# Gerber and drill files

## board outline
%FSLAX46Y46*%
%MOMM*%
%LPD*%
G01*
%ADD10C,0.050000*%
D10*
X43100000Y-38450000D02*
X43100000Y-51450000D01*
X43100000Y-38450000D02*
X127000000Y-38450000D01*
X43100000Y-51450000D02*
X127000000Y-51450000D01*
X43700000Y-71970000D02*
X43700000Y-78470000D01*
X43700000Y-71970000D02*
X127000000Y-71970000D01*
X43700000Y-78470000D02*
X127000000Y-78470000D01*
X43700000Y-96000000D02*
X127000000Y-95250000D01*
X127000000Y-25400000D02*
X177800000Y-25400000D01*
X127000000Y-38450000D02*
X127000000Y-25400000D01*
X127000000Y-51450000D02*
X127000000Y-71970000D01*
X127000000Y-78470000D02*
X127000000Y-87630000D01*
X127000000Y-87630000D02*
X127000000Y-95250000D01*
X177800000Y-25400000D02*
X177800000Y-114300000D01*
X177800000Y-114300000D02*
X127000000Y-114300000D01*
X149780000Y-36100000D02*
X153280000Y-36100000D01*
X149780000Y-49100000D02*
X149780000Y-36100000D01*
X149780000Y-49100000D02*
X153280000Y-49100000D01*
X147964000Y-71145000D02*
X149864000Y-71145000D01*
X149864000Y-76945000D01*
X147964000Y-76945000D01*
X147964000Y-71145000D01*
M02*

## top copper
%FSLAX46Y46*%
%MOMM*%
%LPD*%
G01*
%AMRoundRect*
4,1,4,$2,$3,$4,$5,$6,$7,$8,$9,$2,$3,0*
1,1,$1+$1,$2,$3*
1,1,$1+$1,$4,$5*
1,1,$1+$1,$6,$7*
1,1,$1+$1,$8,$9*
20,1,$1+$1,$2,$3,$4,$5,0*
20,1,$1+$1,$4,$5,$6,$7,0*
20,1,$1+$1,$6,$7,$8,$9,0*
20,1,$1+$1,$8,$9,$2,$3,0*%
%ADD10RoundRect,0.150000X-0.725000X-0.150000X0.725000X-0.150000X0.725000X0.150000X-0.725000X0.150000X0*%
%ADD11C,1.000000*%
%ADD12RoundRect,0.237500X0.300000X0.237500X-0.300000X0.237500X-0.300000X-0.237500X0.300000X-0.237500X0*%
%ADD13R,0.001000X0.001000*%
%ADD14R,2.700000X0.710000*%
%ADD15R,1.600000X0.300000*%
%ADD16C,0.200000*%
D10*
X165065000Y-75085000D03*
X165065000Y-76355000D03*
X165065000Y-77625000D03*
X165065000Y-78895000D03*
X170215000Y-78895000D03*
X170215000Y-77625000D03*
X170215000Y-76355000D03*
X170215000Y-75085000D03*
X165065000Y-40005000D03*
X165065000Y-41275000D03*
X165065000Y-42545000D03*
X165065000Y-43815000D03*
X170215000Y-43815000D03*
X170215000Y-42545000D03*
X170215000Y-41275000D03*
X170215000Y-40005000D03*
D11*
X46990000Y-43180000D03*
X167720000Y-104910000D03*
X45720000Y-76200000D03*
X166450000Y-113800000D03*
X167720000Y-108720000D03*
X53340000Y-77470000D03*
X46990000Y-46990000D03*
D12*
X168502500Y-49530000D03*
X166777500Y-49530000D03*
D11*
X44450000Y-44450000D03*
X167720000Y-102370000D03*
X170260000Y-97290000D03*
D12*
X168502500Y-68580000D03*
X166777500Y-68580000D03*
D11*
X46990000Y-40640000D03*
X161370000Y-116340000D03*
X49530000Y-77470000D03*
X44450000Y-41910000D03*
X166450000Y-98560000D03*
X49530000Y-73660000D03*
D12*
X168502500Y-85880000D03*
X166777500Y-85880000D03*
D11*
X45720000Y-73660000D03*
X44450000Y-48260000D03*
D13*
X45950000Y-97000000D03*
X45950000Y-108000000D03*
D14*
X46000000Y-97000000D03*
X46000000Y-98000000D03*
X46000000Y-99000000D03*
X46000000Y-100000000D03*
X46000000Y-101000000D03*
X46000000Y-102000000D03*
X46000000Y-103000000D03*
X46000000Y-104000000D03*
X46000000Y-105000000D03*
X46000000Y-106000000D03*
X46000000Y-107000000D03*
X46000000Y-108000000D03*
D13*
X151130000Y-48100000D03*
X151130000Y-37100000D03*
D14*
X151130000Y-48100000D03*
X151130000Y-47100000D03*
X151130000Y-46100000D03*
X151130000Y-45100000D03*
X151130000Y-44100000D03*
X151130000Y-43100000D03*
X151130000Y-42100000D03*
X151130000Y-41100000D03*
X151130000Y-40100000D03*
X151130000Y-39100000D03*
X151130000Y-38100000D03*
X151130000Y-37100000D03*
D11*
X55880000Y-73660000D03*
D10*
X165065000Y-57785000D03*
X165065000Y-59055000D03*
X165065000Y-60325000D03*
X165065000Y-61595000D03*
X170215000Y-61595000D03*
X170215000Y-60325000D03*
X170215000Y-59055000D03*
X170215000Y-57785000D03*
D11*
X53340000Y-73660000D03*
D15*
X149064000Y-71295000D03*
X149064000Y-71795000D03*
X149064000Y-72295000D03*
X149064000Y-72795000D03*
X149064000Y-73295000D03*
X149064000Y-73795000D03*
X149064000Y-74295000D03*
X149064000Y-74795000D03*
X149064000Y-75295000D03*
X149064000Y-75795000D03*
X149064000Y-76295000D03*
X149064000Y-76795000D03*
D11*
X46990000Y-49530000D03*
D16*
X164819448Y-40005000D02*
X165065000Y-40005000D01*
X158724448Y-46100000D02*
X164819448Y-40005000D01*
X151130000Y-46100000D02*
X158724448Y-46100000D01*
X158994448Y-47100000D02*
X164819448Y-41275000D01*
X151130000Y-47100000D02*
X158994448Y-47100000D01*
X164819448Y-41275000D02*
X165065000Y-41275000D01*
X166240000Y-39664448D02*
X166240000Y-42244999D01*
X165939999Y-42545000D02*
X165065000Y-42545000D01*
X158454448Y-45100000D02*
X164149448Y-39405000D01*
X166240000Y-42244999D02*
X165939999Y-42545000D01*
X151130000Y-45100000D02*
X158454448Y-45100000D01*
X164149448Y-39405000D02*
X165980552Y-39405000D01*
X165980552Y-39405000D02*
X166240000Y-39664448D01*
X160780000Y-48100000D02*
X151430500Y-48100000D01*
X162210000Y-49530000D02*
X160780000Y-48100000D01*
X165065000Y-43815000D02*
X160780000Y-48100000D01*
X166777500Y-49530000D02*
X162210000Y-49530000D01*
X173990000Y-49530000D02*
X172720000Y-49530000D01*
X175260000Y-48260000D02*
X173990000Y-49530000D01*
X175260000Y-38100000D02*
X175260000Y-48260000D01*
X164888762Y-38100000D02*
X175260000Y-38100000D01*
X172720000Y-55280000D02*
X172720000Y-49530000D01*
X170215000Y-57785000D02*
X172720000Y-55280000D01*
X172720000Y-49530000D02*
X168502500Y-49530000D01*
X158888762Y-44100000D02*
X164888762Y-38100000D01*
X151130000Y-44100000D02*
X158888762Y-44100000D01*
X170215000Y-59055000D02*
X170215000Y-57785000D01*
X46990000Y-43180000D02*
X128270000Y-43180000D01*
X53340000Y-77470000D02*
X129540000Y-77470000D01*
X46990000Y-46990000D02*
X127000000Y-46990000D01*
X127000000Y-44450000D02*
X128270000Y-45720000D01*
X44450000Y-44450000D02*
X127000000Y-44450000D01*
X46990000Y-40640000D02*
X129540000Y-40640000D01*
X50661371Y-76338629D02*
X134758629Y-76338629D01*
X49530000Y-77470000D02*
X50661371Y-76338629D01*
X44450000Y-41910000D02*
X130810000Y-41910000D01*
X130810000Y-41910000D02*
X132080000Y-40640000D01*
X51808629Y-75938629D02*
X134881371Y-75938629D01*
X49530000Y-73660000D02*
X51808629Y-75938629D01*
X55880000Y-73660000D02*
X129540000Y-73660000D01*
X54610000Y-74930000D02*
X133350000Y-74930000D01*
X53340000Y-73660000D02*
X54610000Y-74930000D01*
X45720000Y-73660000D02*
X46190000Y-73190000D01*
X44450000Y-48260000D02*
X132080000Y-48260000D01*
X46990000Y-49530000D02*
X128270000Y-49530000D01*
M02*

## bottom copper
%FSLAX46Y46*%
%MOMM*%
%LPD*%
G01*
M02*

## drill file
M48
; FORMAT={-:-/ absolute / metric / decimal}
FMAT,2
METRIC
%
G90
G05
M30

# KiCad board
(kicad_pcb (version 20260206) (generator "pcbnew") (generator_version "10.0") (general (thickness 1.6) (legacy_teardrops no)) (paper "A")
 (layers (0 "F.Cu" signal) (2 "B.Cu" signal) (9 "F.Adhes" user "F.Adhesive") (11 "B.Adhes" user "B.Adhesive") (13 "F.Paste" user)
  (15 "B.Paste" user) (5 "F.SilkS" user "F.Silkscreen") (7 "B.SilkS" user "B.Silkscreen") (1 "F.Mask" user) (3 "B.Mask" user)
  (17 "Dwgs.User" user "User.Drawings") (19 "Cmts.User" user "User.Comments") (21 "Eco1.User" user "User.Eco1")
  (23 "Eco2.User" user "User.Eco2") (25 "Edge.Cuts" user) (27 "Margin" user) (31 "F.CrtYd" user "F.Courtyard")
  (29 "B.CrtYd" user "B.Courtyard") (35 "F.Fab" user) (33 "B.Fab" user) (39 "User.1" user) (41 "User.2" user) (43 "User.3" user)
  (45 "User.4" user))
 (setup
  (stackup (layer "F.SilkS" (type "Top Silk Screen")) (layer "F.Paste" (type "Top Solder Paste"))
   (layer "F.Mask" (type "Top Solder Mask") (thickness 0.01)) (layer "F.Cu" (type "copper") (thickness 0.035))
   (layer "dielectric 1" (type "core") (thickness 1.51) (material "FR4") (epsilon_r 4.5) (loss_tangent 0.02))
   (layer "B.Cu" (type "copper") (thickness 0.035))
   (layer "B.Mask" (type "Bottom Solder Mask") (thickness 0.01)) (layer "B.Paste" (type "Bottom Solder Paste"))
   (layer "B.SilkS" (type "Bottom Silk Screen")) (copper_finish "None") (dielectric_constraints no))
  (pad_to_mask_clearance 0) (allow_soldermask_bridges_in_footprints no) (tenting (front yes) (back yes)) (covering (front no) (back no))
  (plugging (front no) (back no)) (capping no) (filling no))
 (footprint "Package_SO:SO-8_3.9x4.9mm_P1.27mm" (layer "F.Cu") (at 167.64 76.99)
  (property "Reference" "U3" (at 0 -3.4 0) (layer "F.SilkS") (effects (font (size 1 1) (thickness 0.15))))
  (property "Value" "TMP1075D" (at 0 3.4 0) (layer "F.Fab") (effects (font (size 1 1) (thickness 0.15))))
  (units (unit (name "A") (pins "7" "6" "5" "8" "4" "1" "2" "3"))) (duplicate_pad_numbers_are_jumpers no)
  (pad "1" smd roundrect (at -2.575 -1.905) (size 1.75 0.6) (layers "F.Cu" "F.Mask" "F.Paste") (roundrect_rratio 0.25) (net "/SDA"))
  (pad "2" smd roundrect (at -2.575 -0.635) (size 1.75 0.6) (layers "F.Cu" "F.Mask" "F.Paste") (roundrect_rratio 0.25) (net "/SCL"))
  (pad "3" smd roundrect (at -2.575 0.635) (size 1.75 0.6) (layers "F.Cu" "F.Mask" "F.Paste") (roundrect_rratio 0.25) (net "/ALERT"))
  (pad "4" smd roundrect (at -2.575 1.905) (size 1.75 0.6) (layers "F.Cu" "F.Mask" "F.Paste") (roundrect_rratio 0.25) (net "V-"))
  (pad "5" smd roundrect (at 2.575 1.905) (size 1.75 0.6) (layers "F.Cu" "F.Mask" "F.Paste") (roundrect_rratio 0.25) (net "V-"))
  (pad "6" smd roundrect (at 2.575 0.635) (size 1.75 0.6) (layers "F.Cu" "F.Mask" "F.Paste") (roundrect_rratio 0.25) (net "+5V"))
  (pad "7" smd roundrect (at 2.575 -0.635) (size 1.75 0.6) (layers "F.Cu" "F.Mask" "F.Paste") (roundrect_rratio 0.25) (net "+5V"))
  (pad "8" smd roundrect (at 2.575 -1.905) (size 1.75 0.6) (layers "F.Cu" "F.Mask" "F.Paste") (roundrect_rratio 0.25) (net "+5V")))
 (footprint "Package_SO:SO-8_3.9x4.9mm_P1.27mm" (layer "F.Cu") (at 167.64 41.91)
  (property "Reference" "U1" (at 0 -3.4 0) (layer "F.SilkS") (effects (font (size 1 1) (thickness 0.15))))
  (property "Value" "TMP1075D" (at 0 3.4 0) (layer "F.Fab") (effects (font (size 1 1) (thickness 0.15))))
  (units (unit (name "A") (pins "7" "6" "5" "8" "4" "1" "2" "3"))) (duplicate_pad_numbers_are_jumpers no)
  (pad "1" smd roundrect (at -2.575 -1.905) (size 1.75 0.6) (layers "F.Cu" "F.Mask" "F.Paste") (roundrect_rratio 0.25) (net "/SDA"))
  (pad "2" smd roundrect (at -2.575 -0.635) (size 1.75 0.6) (layers "F.Cu" "F.Mask" "F.Paste") (roundrect_rratio 0.25) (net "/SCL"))
  (pad "3" smd roundrect (at -2.575 0.635) (size 1.75 0.6) (layers "F.Cu" "F.Mask" "F.Paste") (roundrect_rratio 0.25) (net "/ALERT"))
  (pad "4" smd roundrect (at -2.575 1.905) (size 1.75 0.6) (layers "F.Cu" "F.Mask" "F.Paste") (roundrect_rratio 0.25) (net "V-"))
  (pad "5" smd roundrect (at 2.575 1.905) (size 1.75 0.6) (layers "F.Cu" "F.Mask" "F.Paste") (roundrect_rratio 0.25) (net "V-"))
  (pad "6" smd roundrect (at 2.575 0.635) (size 1.75 0.6) (layers "F.Cu" "F.Mask" "F.Paste") (roundrect_rratio 0.25) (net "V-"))
  (pad "7" smd roundrect (at 2.575 -0.635) (size 1.75 0.6) (layers "F.Cu" "F.Mask" "F.Paste") (roundrect_rratio 0.25) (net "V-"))
  (pad "8" smd roundrect (at 2.575 -1.905) (size 1.75 0.6) (layers "F.Cu" "F.Mask" "F.Paste") (roundrect_rratio 0.25) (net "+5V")))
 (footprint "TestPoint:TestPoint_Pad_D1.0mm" (layer "F.Cu") (at 46.99 43.18)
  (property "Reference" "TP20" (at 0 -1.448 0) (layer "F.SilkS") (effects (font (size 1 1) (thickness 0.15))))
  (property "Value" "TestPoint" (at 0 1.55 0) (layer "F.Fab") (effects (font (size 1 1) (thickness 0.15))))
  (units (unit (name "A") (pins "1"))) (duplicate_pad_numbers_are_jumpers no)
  (pad "1" smd circle (at 0 0) (size 1 1) (layers "F.Cu" "F.Mask") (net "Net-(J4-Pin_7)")))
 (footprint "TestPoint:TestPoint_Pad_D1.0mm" (layer "F.Cu") (at 167.72 104.91 90)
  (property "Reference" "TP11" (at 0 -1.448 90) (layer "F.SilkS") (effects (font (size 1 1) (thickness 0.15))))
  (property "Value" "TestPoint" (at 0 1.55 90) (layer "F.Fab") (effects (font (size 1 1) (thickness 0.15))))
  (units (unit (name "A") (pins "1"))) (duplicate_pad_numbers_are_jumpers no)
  (pad "1" smd circle (at 0 0 90) (size 1 1) (layers "F.Cu" "F.Mask") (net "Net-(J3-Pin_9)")))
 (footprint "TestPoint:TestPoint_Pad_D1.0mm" (layer "F.Cu") (at 45.72 76.2)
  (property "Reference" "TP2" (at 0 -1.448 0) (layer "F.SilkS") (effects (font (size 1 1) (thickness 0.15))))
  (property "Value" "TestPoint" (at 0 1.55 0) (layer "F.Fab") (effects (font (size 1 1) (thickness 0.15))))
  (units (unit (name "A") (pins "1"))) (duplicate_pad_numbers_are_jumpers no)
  (pad "1" smd circle (at 0 0) (size 1 1) (layers "F.Cu" "F.Mask") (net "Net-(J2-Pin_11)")))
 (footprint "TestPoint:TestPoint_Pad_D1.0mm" (layer "F.Cu") (at 166.45 113.8 90)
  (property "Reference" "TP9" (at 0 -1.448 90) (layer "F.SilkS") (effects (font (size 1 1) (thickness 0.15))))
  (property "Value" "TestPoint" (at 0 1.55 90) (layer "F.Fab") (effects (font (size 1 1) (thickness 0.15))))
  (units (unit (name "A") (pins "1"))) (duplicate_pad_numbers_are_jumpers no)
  (pad "1" smd circle (at 0 0 90) (size 1 1) (layers "F.Cu" "F.Mask") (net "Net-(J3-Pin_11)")))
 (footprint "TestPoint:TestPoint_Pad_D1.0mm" (layer "F.Cu") (at 167.72 108.72 90)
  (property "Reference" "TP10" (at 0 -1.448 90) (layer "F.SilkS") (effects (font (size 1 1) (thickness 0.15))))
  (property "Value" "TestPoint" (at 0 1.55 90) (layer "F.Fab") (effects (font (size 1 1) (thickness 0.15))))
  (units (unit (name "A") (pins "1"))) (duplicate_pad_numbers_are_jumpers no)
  (pad "1" smd circle (at 0 0 90) (size 1 1) (layers "F.Cu" "F.Mask") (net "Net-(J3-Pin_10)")))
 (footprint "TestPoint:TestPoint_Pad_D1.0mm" (layer "F.Cu") (at 53.34 77.47)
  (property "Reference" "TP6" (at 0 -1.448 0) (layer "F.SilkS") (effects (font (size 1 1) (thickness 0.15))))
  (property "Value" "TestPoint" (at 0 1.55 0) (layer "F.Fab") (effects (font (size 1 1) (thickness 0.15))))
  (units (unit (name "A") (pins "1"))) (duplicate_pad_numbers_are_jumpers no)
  (pad "1" smd circle (at 0 0) (size 1 1) (layers "F.Cu" "F.Mask") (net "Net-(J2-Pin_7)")))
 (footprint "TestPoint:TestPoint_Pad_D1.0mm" (layer "F.Cu") (at 46.99 46.99)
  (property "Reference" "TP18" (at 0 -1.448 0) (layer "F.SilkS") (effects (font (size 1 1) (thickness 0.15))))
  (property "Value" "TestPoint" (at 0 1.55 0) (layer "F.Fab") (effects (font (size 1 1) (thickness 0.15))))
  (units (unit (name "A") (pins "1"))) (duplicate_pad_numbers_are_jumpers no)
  (pad "1" smd circle (at 0 0) (size 1 1) (layers "F.Cu" "F.Mask") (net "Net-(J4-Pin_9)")))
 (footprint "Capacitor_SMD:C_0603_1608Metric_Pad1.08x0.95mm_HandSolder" (layer "F.Cu") (at 167.64 49.53 180)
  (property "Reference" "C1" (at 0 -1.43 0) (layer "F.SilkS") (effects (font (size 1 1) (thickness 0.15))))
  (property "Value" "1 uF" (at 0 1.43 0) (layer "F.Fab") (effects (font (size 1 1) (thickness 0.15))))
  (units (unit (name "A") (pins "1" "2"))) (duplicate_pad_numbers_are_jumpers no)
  (pad "1" smd roundrect (at -0.8625 0 180) (size 1.075 0.95) (layers "F.Cu" "F.Mask" "F.Paste") (roundrect_rratio 0.25) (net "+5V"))
  (pad "2" smd roundrect (at 0.8625 0 180) (size 1.075 0.95) (layers "F.Cu" "F.Mask" "F.Paste") (roundrect_rratio 0.25) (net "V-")))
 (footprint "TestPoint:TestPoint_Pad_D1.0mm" (layer "F.Cu") (at 44.45 44.45)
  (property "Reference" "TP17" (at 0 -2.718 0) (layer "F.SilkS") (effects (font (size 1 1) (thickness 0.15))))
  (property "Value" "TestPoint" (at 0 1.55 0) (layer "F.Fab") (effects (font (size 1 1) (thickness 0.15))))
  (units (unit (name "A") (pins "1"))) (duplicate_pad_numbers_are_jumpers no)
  (pad "1" smd circle (at 0 0) (size 1 1) (layers "F.Cu" "F.Mask") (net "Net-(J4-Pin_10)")))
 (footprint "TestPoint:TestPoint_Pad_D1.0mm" (layer "F.Cu") (at 167.72 102.37 90)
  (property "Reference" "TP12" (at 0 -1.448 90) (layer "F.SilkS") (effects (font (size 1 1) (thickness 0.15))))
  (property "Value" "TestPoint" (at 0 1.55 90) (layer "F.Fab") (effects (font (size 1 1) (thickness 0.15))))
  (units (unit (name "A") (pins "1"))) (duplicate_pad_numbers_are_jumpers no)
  (pad "1" smd circle (at 0 0 90) (size 1 1) (layers "F.Cu" "F.Mask") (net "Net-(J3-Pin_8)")))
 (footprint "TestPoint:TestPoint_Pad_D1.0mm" (layer "F.Cu") (at 170.26 97.29 90)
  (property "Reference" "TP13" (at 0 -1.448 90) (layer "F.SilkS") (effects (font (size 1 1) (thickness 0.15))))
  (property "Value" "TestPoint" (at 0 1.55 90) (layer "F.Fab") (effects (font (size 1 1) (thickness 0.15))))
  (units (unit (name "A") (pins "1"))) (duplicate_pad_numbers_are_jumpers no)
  (pad "1" smd circle (at 0 0 90) (size 1 1) (layers "F.Cu" "F.Mask") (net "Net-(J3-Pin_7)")))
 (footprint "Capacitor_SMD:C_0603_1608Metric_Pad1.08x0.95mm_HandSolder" (layer "F.Cu") (at 167.64 68.58 180)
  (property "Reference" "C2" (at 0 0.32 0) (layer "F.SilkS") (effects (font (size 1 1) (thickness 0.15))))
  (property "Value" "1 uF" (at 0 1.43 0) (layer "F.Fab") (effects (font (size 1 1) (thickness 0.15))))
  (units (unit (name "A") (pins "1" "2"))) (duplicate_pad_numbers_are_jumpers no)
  (pad "1" smd roundrect (at -0.8625 0 180) (size 1.075 0.95) (layers "F.Cu" "F.Mask" "F.Paste") (roundrect_rratio 0.25) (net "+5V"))
  (pad "2" smd roundrect (at 0.8625 0 180) (size 1.075 0.95) (layers "F.Cu" "F.Mask" "F.Paste") (roundrect_rratio 0.25) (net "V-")))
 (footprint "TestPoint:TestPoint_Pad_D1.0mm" (layer "F.Cu") (at 46.99 40.64)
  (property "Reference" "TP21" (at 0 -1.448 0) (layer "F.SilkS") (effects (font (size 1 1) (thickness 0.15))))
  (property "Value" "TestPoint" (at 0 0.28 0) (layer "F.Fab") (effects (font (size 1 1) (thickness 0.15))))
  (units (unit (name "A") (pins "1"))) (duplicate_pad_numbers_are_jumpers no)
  (pad "1" smd circle (at 0 0) (size 1 1) (layers "F.Cu" "F.Mask") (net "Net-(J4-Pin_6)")))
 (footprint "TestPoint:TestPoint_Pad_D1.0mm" (layer "F.Cu") (at 161.37 116.34 90)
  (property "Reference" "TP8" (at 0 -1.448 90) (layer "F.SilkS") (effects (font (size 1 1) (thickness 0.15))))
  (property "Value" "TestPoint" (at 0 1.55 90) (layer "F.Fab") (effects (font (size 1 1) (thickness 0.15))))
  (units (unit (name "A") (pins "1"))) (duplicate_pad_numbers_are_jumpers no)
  (pad "1" smd circle (at 0 0 90) (size 1 1) (layers "F.Cu" "F.Mask") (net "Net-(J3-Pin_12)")))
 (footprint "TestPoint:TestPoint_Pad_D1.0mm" (layer "F.Cu") (at 49.53 77.47)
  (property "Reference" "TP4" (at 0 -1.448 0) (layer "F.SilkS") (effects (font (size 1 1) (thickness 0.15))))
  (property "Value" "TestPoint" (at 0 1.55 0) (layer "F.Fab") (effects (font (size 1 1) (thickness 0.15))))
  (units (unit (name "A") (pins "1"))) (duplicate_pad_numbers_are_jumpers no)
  (pad "1" smd circle (at 0 0) (size 1 1) (layers "F.Cu" "F.Mask") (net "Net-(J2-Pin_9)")))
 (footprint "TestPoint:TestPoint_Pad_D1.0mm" (layer "F.Cu") (at 44.45 41.91)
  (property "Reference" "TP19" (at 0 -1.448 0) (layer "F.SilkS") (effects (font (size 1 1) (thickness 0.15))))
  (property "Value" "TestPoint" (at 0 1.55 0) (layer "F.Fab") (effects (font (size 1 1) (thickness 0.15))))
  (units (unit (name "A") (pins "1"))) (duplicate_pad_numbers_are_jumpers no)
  (pad "1" smd circle (at 0 0) (size 1 1) (layers "F.Cu" "F.Mask") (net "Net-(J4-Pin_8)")))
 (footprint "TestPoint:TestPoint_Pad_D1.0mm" (layer "F.Cu") (at 166.45 98.56 90)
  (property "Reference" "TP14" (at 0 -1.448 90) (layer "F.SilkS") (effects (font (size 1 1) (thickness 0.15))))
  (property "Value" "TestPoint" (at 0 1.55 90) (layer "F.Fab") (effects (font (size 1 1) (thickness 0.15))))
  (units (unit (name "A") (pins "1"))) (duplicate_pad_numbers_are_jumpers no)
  (pad "1" smd circle (at 0 0 90) (size 1 1) (layers "F.Cu" "F.Mask") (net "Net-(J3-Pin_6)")))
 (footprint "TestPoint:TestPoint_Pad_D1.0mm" (layer "F.Cu") (at 49.53 73.66)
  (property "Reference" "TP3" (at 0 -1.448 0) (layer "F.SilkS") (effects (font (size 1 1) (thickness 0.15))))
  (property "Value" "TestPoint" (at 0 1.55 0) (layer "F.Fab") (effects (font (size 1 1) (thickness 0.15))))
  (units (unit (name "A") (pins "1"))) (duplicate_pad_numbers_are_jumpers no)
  (pad "1" smd circle (at 0 0) (size 1 1) (layers "F.Cu" "F.Mask") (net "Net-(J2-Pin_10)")))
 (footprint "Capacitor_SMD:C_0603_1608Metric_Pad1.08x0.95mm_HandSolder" (layer "F.Cu") (at 167.64 85.88 180)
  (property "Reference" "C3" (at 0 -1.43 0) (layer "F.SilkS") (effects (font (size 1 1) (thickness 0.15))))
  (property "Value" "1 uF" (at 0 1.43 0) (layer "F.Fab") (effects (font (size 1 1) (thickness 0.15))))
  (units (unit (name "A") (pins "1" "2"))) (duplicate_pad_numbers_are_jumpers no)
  (pad "1" smd roundrect (at -0.8625 0 180) (size 1.075 0.95) (layers "F.Cu" "F.Mask" "F.Paste") (roundrect_rratio 0.25) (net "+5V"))
  (pad "2" smd roundrect (at 0.8625 0 180) (size 1.075 0.95) (layers "F.Cu" "F.Mask" "F.Paste") (roundrect_rratio 0.25) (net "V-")))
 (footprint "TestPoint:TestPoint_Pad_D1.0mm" (layer "F.Cu") (at 45.72 73.66)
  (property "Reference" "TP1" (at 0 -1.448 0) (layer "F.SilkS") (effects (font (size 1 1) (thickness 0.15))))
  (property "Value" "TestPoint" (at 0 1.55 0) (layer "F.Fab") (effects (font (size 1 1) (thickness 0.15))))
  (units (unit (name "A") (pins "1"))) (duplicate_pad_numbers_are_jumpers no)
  (pad "1" smd circle (at 0 0) (size 1 1) (layers "F.Cu" "F.Mask") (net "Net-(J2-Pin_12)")))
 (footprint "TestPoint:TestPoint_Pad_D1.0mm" (layer "F.Cu") (at 44.45 48.26)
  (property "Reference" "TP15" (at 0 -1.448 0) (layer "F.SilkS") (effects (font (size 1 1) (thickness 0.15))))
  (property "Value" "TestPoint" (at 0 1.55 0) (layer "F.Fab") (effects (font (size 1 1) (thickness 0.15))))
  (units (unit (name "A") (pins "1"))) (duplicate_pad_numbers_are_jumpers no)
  (pad "1" smd circle (at 0 0) (size 1 1) (layers "F.Cu" "F.Mask") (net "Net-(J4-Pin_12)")))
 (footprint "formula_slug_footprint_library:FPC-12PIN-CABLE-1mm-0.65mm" (layer "F.Cu") (at 47.35 102.5 -90)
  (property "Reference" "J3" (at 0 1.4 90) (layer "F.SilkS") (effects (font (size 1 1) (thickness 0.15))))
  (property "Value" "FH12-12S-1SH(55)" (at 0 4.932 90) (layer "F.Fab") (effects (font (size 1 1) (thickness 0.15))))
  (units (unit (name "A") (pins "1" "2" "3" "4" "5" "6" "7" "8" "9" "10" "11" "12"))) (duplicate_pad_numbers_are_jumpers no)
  (pad "0" smd rect (at -5.5 1.4 270) (size 0.001 0.001) (layers "F.Cu" "F.Mask" "F.Paste") (thermal_bridge_angle 45))
  (pad "0" smd rect (at 5.5 1.4 270) (size 0.001 0.001) (layers "F.Cu" "F.Mask" "F.Paste") (thermal_bridge_angle 45))
  (pad "1" smd rect (at -5.5 1.35 270) (size 0.71 2.7) (layers "F.Cu" "F.Mask" "F.Paste") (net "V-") (thermal_bridge_angle 45))
  (pad "2" smd rect (at -4.5 1.35 270) (size 0.71 2.7) (layers "F.Cu" "F.Mask" "F.Paste") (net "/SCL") (thermal_bridge_angle 45))
  (pad "3" smd rect (at -3.5 1.35 270) (size 0.71 2.7) (layers "F.Cu" "F.Mask" "F.Paste") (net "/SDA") (thermal_bridge_angle 45))
  (pad "4" smd rect (at -2.5 1.35 270) (size 0.71 2.7) (layers "F.Cu" "F.Mask" "F.Paste") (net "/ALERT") (thermal_bridge_angle 45))
  (pad "5" smd rect (at -1.5 1.35 270) (size 0.71 2.7) (layers "F.Cu" "F.Mask" "F.Paste") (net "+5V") (thermal_bridge_angle 45))
  (pad "6" smd rect (at -0.5 1.35 270) (size 0.71 2.7) (layers "F.Cu" "F.Mask" "F.Paste") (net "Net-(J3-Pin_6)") (thermal_bridge_angle 45))
  (pad "7" smd rect (at 0.5 1.35 270) (size 0.71 2.7) (layers "F.Cu" "F.Mask" "F.Paste") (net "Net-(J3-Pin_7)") (thermal_bridge_angle 45))
  (pad "8" smd rect (at 1.5 1.35 270) (size 0.71 2.7) (layers "F.Cu" "F.Mask" "F.Paste") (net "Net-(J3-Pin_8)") (thermal_bridge_angle 45))
  (pad "9" smd rect (at 2.5 1.35 270) (size 0.71 2.7) (layers "F.Cu" "F.Mask" "F.Paste") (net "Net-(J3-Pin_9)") (thermal_bridge_angle 45))
  (pad "10" smd rect (at 3.5 1.35 270) (size 0.71 2.7) (layers "F.Cu" "F.Mask" "F.Paste") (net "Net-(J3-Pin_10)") (thermal_bridge_angle 45))
  (pad "11" smd rect (at 4.5 1.35 270) (size 0.71 2.7) (layers "F.Cu" "F.Mask" "F.Paste") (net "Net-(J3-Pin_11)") (thermal_bridge_angle 45))
  (pad "12" smd rect (at 5.5 1.35 270) (size 0.71 2.7) (layers "F.Cu" "F.Mask" "F.Paste") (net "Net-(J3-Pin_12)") (thermal_bridge_angle 45)))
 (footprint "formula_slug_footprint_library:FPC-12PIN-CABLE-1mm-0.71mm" (layer "F.Cu") (at 149.78 42.6 90)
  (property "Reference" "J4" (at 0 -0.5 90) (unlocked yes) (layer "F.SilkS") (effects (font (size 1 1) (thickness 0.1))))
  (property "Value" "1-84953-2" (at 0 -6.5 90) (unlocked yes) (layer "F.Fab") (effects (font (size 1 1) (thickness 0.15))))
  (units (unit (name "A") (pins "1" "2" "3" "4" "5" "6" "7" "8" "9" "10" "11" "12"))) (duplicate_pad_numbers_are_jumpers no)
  (fp_line (start 6.5 0) (end 6.5 3.5) (stroke (width 0.05) (type solid)) (layer "Edge.Cuts"))
  (fp_line (start -6.5 0) (end 6.5 0) (stroke (width 0.05) (type solid)) (layer "Edge.Cuts"))
  (fp_line (start -6.5 0) (end -6.5 3.5) (stroke (width 0.05) (type solid)) (layer "Edge.Cuts"))
  (pad "0" smd rect (at -5.5 1.35 90) (size 0.001 0.001) (layers "F.Cu" "F.Mask" "F.Paste") (thermal_bridge_angle 45))
  (pad "0" smd rect (at 5.5 1.35 90) (size 0.001 0.001) (layers "F.Cu" "F.Mask" "F.Paste") (thermal_bridge_angle 45))
  (pad "1" smd rect (at -5.5 1.35 90) (size 0.71 2.7) (layers "F.Cu" "F.Mask" "F.Paste") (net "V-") (thermal_bridge_angle 45))
  (pad "2" smd rect (at -4.5 1.35 90) (size 0.71 2.7) (layers "F.Cu" "F.Mask" "F.Paste") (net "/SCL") (thermal_bridge_angle 45))
  (pad "3" smd rect (at -3.5 1.35 90) (size 0.71 2.7) (layers "F.Cu" "F.Mask" "F.Paste") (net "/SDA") (thermal_bridge_angle 45))
  (pad "4" smd rect (at -2.5 1.35 90) (size 0.71 2.7) (layers "F.Cu" "F.Mask" "F.Paste") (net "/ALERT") (thermal_bridge_angle 45))
  (pad "5" smd rect (at -1.5 1.35 90) (size 0.71 2.7) (layers "F.Cu" "F.Mask" "F.Paste") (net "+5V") (thermal_bridge_angle 45))
  (pad "6" smd rect (at -0.5 1.35 90) (size 0.71 2.7) (layers "F.Cu" "F.Mask" "F.Paste") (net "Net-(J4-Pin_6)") (thermal_bridge_angle 45))
  (pad "7" smd rect (at 0.5 1.35 90) (size 0.71 2.7) (layers "F.Cu" "F.Mask" "F.Paste") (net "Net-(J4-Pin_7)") (thermal_bridge_angle 45))
  (pad "8" smd rect (at 1.5 1.35 90) (size 0.71 2.7) (layers "F.Cu" "F.Mask" "F.Paste") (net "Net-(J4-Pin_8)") (thermal_bridge_angle 45))
  (pad "9" smd rect (at 2.5 1.35 90) (size 0.71 2.7) (layers "F.Cu" "F.Mask" "F.Paste") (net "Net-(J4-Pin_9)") (thermal_bridge_angle 45))
  (pad "10" smd rect (at 3.5 1.35 90) (size 0.71 2.7) (layers "F.Cu" "F.Mask" "F.Paste") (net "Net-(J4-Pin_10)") (thermal_bridge_angle 45))
  (pad "11" smd rect (at 4.5 1.35 90) (size 0.71 2.7) (layers "F.Cu" "F.Mask" "F.Paste") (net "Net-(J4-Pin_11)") (thermal_bridge_angle 45))
  (pad "12" smd rect (at 5.5 1.35 90) (size 0.71 2.7) (layers "F.Cu" "F.Mask" "F.Paste") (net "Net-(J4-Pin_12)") (thermal_bridge_angle 45)))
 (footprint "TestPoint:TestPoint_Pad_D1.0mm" (layer "F.Cu") (at 55.88 73.66)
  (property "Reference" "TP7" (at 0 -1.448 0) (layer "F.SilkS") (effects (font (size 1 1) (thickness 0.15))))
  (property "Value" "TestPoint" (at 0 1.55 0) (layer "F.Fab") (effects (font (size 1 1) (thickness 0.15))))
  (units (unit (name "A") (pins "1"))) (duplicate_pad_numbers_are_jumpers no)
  (pad "1" smd circle (at 0 0) (size 1 1) (layers "F.Cu" "F.Mask") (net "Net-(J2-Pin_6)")))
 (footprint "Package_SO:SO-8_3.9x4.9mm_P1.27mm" (layer "F.Cu") (at 167.64 59.69)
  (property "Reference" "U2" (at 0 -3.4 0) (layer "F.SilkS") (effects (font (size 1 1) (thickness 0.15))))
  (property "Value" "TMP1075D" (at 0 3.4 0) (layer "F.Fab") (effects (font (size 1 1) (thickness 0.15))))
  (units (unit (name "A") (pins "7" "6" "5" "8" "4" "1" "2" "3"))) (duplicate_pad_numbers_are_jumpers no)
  (pad "1" smd roundrect (at -2.575 -1.905) (size 1.75 0.6) (layers "F.Cu" "F.Mask" "F.Paste") (roundrect_rratio 0.25) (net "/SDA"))
  (pad "2" smd roundrect (at -2.575 -0.635) (size 1.75 0.6) (layers "F.Cu" "F.Mask" "F.Paste") (roundrect_rratio 0.25) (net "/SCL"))
  (pad "3" smd roundrect (at -2.575 0.635) (size 1.75 0.6) (layers "F.Cu" "F.Mask" "F.Paste") (roundrect_rratio 0.25) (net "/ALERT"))
  (pad "4" smd roundrect (at -2.575 1.905) (size 1.75 0.6) (layers "F.Cu" "F.Mask" "F.Paste") (roundrect_rratio 0.25) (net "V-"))
  (pad "5" smd roundrect (at 2.575 1.905) (size 1.75 0.6) (layers "F.Cu" "F.Mask" "F.Paste") (roundrect_rratio 0.25) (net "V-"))
  (pad "6" smd roundrect (at 2.575 0.635) (size 1.75 0.6) (layers "F.Cu" "F.Mask" "F.Paste") (roundrect_rratio 0.25) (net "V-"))
  (pad "7" smd roundrect (at 2.575 -0.635) (size 1.75 0.6) (layers "F.Cu" "F.Mask" "F.Paste") (roundrect_rratio 0.25) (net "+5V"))
  (pad "8" smd roundrect (at 2.575 -1.905) (size 1.75 0.6) (layers "F.Cu" "F.Mask" "F.Paste") (roundrect_rratio 0.25) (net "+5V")))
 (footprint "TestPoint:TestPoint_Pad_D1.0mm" (layer "F.Cu") (at 53.34 73.66)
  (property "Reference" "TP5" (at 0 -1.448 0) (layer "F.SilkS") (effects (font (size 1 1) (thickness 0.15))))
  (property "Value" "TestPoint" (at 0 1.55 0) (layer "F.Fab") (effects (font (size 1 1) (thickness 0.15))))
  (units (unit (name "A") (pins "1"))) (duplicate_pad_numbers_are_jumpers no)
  (pad "1" smd circle (at 0 0) (size 1 1) (layers "F.Cu" "F.Mask") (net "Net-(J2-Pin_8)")))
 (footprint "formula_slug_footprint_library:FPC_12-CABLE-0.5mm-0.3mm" (layer "F.Cu") (at 149.864 74.045 -90)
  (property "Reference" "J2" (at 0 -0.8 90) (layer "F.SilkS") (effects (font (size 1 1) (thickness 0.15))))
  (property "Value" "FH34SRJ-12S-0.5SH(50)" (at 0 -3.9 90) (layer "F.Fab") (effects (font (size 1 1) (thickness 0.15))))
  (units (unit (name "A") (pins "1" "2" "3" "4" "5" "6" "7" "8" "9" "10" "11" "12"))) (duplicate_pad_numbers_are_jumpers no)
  (fp_rect (start -2.9 0) (end 2.9 1.9) (stroke (width 0.05) (type solid)) (fill no) (layer "Edge.Cuts"))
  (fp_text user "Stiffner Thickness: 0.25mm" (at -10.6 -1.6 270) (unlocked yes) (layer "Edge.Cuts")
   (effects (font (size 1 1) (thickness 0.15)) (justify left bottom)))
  (pad "1" smd rect (at -2.75 0.8 270) (size 0.3 1.6) (layers "F.Cu" "F.Mask" "F.Paste") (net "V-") (thermal_bridge_angle 45))
  (pad "2" smd rect (at -2.25 0.8 270) (size 0.3 1.6) (layers "F.Cu" "F.Mask" "F.Paste") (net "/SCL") (thermal_bridge_angle 45))
  (pad "3" smd rect (at -1.75 0.8 270) (size 0.3 1.6) (layers "F.Cu" "F.Mask" "F.Paste") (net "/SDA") (thermal_bridge_angle 45))
  (pad "4" smd rect (at -1.25 0.8 270) (size 0.3 1.6) (layers "F.Cu" "F.Mask" "F.Paste") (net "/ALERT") (thermal_bridge_angle 45))
  (pad "5" smd rect (at -0.75 0.8 270) (size 0.3 1.6) (layers "F.Cu" "F.Mask" "F.Paste") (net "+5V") (thermal_bridge_angle 45))
  (pad "6" smd rect (at -0.25 0.8 270) (size 0.3 1.6) (layers "F.Cu" "F.Mask" "F.Paste") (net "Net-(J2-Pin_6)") (thermal_bridge_angle 45))
  (pad "7" smd rect (at 0.25 0.8 270) (size 0.3 1.6) (layers "F.Cu" "F.Mask" "F.Paste") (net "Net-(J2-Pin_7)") (thermal_bridge_angle 45))
  (pad "8" smd rect (at 0.75 0.8 270) (size 0.3 1.6) (layers "F.Cu" "F.Mask" "F.Paste") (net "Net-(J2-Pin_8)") (thermal_bridge_angle 45))
  (pad "9" smd rect (at 1.25 0.8 270) (size 0.3 1.6) (layers "F.Cu" "F.Mask" "F.Paste") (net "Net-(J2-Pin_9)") (thermal_bridge_angle 45))
  (pad "10" smd rect (at 1.75 0.8 270) (size 0.3 1.6) (layers "F.Cu" "F.Mask" "F.Paste") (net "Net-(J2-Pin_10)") (thermal_bridge_angle 45))
  (pad "11" smd rect (at 2.25 0.8 270) (size 0.3 1.6) (layers "F.Cu" "F.Mask" "F.Paste") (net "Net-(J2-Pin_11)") (thermal_bridge_angle 45))
  (pad "12" smd rect (at 2.75 0.8 270) (size 0.3 1.6) (layers "F.Cu" "F.Mask" "F.Paste") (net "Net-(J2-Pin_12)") (thermal_bridge_angle 45)))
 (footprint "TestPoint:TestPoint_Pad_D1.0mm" (layer "F.Cu") (at 46.99 49.53)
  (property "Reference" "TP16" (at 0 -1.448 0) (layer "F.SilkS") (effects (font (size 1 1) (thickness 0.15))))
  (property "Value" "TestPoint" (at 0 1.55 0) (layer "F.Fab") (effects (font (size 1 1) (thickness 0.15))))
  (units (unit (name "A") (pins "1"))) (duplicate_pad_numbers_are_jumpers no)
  (pad "1" smd circle (at 0 0) (size 1 1) (layers "F.Cu" "F.Mask") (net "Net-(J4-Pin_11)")))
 (gr_line (start 43.1 38.45) (end 43.1 51.45) (stroke (width 0.05) (type default)) (layer "Edge.Cuts"))
 (gr_line (start 43.1 38.45) (end 127 38.45) (stroke (width 0.05) (type default)) (layer "Edge.Cuts"))
 (gr_line (start 43.1 51.45) (end 127 51.45) (stroke (width 0.05) (type default)) (layer "Edge.Cuts"))
 (gr_line (start 43.7 71.97) (end 43.7 78.47) (stroke (width 0.05) (type default)) (layer "Edge.Cuts"))
 (gr_line (start 43.7 71.97) (end 127 71.97) (stroke (width 0.05) (type default)) (layer "Edge.Cuts"))
 (gr_line (start 43.7 78.47) (end 127 78.47) (stroke (width 0.05) (type default)) (layer "Edge.Cuts"))
 (gr_line (start 43.7 96) (end 127 95.25) (stroke (width 0.05) (type default)) (layer "Edge.Cuts"))
 (gr_line (start 127 25.4) (end 177.8 25.4) (stroke (width 0.05) (type default)) (layer "Edge.Cuts"))
 (gr_line (start 127 38.45) (end 127 25.4) (stroke (width 0.05) (type default)) (layer "Edge.Cuts"))
 (gr_line (start 127 51.45) (end 127 71.97) (stroke (width 0.05) (type default)) (layer "Edge.Cuts"))
 (gr_line (start 127 78.47) (end 127 87.63) (stroke (width 0.05) (type default)) (layer "Edge.Cuts"))
 (gr_line (start 127 87.63) (end 127 95.25) (stroke (width 0.05) (type default)) (layer "Edge.Cuts"))
 (gr_line (start 177.8 25.4) (end 177.8 114.3) (stroke (width 0.05) (type default)) (layer "Edge.Cuts"))
 (gr_line (start 177.8 114.3) (end 127 114.3) (stroke (width 0.05) (type default)) (layer "Edge.Cuts"))
 (segment (start 164.819448 40.005) (end 165.065 40.005) (width 0.2) (layer "F.Cu") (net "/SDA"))
 (segment (start 158.724448 46.1) (end 164.819448 40.005) (width 0.2) (layer "F.Cu") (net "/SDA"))
 (segment (start 151.13 46.1) (end 158.724448 46.1) (width 0.2) (layer "F.Cu") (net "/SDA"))
 (segment (start 158.994448 47.1) (end 164.819448 41.275) (width 0.2) (layer "F.Cu") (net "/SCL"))
 (segment (start 151.13 47.1) (end 158.994448 47.1) (width 0.2) (layer "F.Cu") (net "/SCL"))
 (segment (start 164.819448 41.275) (end 165.065 41.275) (width 0.2) (layer "F.Cu") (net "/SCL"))
 (segment (start 166.24 39.664448) (end 166.24 42.244999) (width 0.2) (layer "F.Cu") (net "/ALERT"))
 (segment (start 165.939999 42.545) (end 165.065 42.545) (width 0.2) (layer "F.Cu") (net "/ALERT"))
 (segment (start 158.454448 45.1) (end 164.149448 39.405) (width 0.2) (layer "F.Cu") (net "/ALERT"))
 (segment (start 166.24 42.244999) (end 165.939999 42.545) (width 0.2) (layer "F.Cu") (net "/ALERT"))
 (segment (start 151.13 45.1) (end 158.454448 45.1) (width 0.2) (layer "F.Cu") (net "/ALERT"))
 (segment (start 164.149448 39.405) (end 165.980552 39.405) (width 0.2) (layer "F.Cu") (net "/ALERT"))
 (segment (start 165.980552 39.405) (end 166.24 39.664448) (width 0.2) (layer "F.Cu") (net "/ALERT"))
 (segment (start 160.78 48.1) (end 151.4305 48.1) (width 0.2) (layer "F.Cu") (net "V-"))
 (segment (start 162.21 49.53) (end 160.78 48.1) (width 0.2) (layer "F.Cu") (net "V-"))
 (segment (start 165.065 43.815) (end 160.78 48.1) (width 0.2) (layer "F.Cu") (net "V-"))
 (segment (start 166.7775 49.53) (end 162.21 49.53) (width 0.2) (layer "F.Cu") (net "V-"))
 (segment (start 173.99 49.53) (end 172.72 49.53) (width 0.2) (layer "F.Cu") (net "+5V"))
 (segment (start 175.26 48.26) (end 173.99 49.53) (width 0.2) (layer "F.Cu") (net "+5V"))
 (segment (start 175.26 38.1) (end 175.26 48.26) (width 0.2) (layer "F.Cu") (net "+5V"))
 (segment (start 164.888762 38.1) (end 175.26 38.1) (width 0.2) (layer "F.Cu") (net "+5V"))
 (segment (start 172.72 55.28) (end 172.72 49.53) (width 0.2) (layer "F.Cu") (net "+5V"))
 (segment (start 170.215 57.785) (end 172.72 55.28) (width 0.2) (layer "F.Cu") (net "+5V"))
 (segment (start 172.72 49.53) (end 168.5025 49.53) (width 0.2) (layer "F.Cu") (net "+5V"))
 (segment (start 158.888762 44.1) (end 164.888762 38.1) (width 0.2) (layer "F.Cu") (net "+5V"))
 (segment (start 151.13 44.1) (end 158.888762 44.1) (width 0.2) (layer "F.Cu") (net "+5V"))
 (segment (start 170.215 59.055) (end 170.215 57.785) (width 0.2) (layer "F.Cu") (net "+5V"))
 (segment (start 46.99 43.18) (end 128.27 43.18) (width 0.2) (layer "F.Cu") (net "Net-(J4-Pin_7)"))
 (segment (start 53.34 77.47) (end 129.54 77.47) (width 0.2) (layer "F.Cu") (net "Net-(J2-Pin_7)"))
 (segment (start 46.99 46.99) (end 127 46.99) (width 0.2) (layer "F.Cu") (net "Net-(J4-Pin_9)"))
 (segment (start 127 44.45) (end 128.27 45.72) (width 0.2) (layer "F.Cu") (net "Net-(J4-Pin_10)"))
 (segment (start 44.45 44.45) (end 127 44.45) (width 0.2) (layer "F.Cu") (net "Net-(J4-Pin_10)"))
 (segment (start 46.99 40.64) (end 129.54 40.64) (width 0.2) (layer "F.Cu") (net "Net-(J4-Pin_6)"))
 (segment (start 50.661371 76.338629) (end 134.758629 76.338629) (width 0.2) (layer "F.Cu") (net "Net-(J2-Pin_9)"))
 (segment (start 49.53 77.47) (end 50.661371 76.338629) (width 0.2) (layer "F.Cu") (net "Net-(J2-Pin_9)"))
 (segment (start 44.45 41.91) (end 130.81 41.91) (width 0.2) (layer "F.Cu") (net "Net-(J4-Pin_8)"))
 (segment (start 130.81 41.91) (end 132.08 40.64) (width 0.2) (layer "F.Cu") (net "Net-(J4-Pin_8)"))
 (segment (start 51.808629 75.938629) (end 134.881371 75.938629) (width 0.2) (layer "F.Cu") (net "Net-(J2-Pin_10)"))
 (segment (start 49.53 73.66) (end 51.808629 75.938629) (width 0.2) (layer "F.Cu") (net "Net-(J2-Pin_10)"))
 (segment (start 55.88 73.66) (end 129.54 73.66) (width 0.2) (layer "F.Cu") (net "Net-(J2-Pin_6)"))
 (segment (start 54.61 74.93) (end 133.35 74.93) (width 0.2) (layer "F.Cu") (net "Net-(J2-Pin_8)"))
 (segment (start 53.34 73.66) (end 54.61 74.93) (width 0.2) (layer "F.Cu") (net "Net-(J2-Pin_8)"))
 (segment (start 45.72 73.66) (end 46.19 73.19) (width 0.2) (layer "F.Cu") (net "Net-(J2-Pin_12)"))
 (segment (start 44.45 48.26) (end 132.08 48.26) (width 0.2) (layer "F.Cu") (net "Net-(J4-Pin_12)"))
 (segment (start 46.99 49.53) (end 128.27 49.53) (width 0.2) (layer "F.Cu") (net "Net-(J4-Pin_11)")))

